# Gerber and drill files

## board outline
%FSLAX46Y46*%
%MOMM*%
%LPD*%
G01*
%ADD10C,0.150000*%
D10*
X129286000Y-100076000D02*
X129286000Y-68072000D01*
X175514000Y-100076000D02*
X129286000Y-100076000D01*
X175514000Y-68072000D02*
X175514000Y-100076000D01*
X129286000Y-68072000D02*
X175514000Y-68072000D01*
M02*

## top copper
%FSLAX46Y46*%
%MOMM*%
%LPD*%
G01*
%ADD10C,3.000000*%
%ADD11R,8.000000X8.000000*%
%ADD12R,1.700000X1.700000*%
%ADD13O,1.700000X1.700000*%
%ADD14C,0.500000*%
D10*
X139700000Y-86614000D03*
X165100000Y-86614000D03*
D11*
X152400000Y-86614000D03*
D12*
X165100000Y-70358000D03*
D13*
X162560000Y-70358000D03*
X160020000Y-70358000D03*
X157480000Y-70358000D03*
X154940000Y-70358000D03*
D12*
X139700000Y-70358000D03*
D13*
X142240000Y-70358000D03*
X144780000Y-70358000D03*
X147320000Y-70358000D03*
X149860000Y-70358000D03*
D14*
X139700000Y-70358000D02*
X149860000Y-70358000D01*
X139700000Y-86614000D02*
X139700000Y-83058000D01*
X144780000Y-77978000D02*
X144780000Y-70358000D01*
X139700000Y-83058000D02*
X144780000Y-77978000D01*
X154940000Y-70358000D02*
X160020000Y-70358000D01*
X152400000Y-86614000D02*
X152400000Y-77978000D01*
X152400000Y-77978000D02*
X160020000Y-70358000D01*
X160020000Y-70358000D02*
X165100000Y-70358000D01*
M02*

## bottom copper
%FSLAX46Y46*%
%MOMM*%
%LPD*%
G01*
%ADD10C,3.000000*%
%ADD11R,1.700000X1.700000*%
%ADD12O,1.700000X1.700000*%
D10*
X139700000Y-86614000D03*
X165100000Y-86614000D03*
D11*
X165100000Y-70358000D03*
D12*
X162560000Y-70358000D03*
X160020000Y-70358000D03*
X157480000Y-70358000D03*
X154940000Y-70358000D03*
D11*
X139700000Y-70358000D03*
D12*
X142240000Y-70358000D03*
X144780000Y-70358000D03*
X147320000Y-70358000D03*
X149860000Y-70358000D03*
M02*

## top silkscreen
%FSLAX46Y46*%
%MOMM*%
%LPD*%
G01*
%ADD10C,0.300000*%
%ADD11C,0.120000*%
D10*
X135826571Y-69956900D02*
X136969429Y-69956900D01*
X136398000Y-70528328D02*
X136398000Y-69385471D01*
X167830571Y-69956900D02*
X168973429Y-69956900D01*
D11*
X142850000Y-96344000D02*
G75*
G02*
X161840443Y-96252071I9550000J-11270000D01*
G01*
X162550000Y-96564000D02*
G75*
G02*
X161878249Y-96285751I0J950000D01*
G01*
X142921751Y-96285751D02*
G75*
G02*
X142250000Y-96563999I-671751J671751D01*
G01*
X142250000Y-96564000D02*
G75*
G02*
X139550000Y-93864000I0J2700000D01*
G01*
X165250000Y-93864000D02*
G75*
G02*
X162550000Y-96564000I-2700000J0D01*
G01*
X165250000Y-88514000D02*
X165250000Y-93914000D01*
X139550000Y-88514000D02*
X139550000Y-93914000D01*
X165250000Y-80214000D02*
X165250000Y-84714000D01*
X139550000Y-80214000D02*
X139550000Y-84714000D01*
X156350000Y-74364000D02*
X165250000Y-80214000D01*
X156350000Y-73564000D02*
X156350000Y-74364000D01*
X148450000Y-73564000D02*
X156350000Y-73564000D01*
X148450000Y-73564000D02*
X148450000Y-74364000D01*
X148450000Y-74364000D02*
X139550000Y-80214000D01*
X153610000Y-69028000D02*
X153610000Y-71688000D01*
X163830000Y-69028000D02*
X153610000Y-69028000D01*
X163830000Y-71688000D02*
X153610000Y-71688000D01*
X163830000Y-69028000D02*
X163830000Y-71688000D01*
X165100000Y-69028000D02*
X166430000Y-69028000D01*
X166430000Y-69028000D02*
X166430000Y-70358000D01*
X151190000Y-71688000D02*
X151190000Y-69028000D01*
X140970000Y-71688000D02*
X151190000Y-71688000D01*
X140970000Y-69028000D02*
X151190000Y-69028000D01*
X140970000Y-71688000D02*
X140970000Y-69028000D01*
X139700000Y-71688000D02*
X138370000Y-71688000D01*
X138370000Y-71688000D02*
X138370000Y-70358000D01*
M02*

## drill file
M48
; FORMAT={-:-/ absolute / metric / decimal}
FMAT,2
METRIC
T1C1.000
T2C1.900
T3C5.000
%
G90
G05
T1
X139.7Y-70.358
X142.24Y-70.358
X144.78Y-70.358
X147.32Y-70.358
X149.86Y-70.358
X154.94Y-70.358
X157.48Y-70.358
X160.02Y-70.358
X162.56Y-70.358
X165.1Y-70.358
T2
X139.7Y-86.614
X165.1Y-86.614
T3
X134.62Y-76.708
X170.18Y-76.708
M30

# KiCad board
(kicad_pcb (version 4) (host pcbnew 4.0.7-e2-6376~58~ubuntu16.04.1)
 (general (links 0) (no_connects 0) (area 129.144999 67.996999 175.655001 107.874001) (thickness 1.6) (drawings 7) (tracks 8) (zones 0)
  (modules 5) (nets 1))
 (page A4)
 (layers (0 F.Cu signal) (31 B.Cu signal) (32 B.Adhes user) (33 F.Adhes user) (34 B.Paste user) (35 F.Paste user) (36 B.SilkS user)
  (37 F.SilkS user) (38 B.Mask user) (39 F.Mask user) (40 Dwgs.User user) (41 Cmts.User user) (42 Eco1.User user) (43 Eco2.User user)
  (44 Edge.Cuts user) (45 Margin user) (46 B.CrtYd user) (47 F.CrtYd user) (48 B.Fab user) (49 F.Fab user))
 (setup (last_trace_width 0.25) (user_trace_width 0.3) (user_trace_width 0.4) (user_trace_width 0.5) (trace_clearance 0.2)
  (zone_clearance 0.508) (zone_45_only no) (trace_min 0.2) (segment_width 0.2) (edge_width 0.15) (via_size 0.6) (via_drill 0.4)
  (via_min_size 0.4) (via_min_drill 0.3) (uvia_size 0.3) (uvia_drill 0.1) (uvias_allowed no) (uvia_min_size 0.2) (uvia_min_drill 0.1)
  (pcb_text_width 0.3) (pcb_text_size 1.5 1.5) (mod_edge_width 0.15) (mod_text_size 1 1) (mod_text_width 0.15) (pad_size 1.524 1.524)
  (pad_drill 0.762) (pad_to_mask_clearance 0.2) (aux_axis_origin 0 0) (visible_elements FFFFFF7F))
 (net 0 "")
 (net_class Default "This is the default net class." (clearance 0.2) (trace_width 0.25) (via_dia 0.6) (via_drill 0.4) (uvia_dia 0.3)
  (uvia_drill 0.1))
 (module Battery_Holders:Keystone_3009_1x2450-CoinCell (layer F.Cu) (at 152.4 86.614)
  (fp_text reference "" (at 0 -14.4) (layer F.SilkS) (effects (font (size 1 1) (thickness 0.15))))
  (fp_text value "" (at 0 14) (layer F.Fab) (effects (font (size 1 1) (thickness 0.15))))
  (fp_arc (start 0 21) (end -9.55 9.73) (angle 80) (layer F.SilkS) (width 0.12))
  (fp_arc (start 10.15 9) (end 10.15 9.95) (angle 45) (layer F.SilkS) (width 0.12))
  (fp_arc (start -10.15 9) (end -10.15 9.95) (angle -45) (layer F.SilkS) (width 0.12))
  (fp_arc (start -10.15 7.25) (end -10.15 9.95) (angle 90) (layer F.SilkS) (width 0.12))
  (fp_arc (start 10.15 7.25) (end 10.15 9.95) (angle -90) (layer F.SilkS) (width 0.12))
  (fp_line (start 12.85 1.9) (end 12.85 7.3) (layer F.SilkS) (width 0.12))
  (fp_line (start -12.85 1.9) (end -12.85 7.3) (layer F.SilkS) (width 0.12))
  (fp_line (start 12.85 -6.4) (end 12.85 -1.9) (layer F.SilkS) (width 0.12))
  (fp_line (start -12.85 -6.4) (end -12.85 -1.9) (layer F.SilkS) (width 0.12))
  (fp_line (start 3.95 -12.25) (end 12.85 -6.4) (layer F.SilkS) (width 0.12))
  (fp_line (start 3.95 -13.05) (end 3.95 -12.25) (layer F.SilkS) (width 0.12))
  (fp_line (start -3.95 -13.05) (end 3.95 -13.05) (layer F.SilkS) (width 0.12))
  (fp_line (start -3.95 -13.05) (end -3.95 -12.25) (layer F.SilkS) (width 0.12))
  (fp_line (start -3.95 -12.25) (end -12.85 -6.4) (layer F.SilkS) (width 0.12))
  (pad 1 thru_hole circle (at -12.7 0) (size 3 3) (drill 1.9) (layers *.Cu *.Mask))
  (pad 1 thru_hole circle (at 12.7 0) (size 3 3) (drill 1.9) (layers *.Cu *.Mask)) (pad 2 smd rect (at 0 0) (size 8 8) (layers F.Cu F.Mask)))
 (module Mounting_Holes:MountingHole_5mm (layer F.Cu) (at 170.18 76.708)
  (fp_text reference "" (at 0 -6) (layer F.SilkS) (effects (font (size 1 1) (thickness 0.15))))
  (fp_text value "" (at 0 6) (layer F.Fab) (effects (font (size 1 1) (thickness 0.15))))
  (pad 1 np_thru_hole circle (at 0 0) (size 5 5) (drill 5) (layers *.Cu *.Mask)))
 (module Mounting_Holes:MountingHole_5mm (layer F.Cu) (at 134.62 76.708)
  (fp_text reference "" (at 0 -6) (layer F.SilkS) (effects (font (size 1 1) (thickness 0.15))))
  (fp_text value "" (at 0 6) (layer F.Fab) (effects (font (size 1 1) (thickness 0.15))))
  (pad 1 np_thru_hole circle (at 0 0) (size 5 5) (drill 5) (layers *.Cu *.Mask)))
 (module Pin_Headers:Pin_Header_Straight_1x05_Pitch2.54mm (layer F.Cu) (at 165.1 70.358 270)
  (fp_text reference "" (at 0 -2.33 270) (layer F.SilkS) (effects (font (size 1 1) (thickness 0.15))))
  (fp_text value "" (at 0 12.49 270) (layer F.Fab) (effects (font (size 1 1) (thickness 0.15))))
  (fp_line (start -1.33 11.49) (end 1.33 11.49) (layer F.SilkS) (width 0.12))
  (fp_line (start -1.33 1.27) (end -1.33 11.49) (layer F.SilkS) (width 0.12))
  (fp_line (start 1.33 1.27) (end 1.33 11.49) (layer F.SilkS) (width 0.12))
  (fp_line (start -1.33 1.27) (end 1.33 1.27) (layer F.SilkS) (width 0.12))
  (fp_line (start -1.33 0) (end -1.33 -1.33) (layer F.SilkS) (width 0.12))
  (fp_line (start -1.33 -1.33) (end 0 -1.33) (layer F.SilkS) (width 0.12))
  (pad 1 thru_hole rect (at 0 0 270) (size 1.7 1.7) (drill 1) (layers *.Cu *.Mask))
  (pad 2 thru_hole oval (at 0 2.54 270) (size 1.7 1.7) (drill 1) (layers *.Cu *.Mask))
  (pad 3 thru_hole oval (at 0 5.08 270) (size 1.7 1.7) (drill 1) (layers *.Cu *.Mask))
  (pad 4 thru_hole oval (at 0 7.62 270) (size 1.7 1.7) (drill 1) (layers *.Cu *.Mask))
  (pad 5 thru_hole oval (at 0 10.16 270) (size 1.7 1.7) (drill 1) (layers *.Cu *.Mask)))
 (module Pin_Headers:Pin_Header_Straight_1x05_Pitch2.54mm (layer F.Cu) (at 139.7 70.358 90)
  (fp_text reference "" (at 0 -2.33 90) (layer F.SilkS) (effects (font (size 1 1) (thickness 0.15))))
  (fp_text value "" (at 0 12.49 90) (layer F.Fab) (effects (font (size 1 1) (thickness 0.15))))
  (fp_line (start -1.33 11.49) (end 1.33 11.49) (layer F.SilkS) (width 0.12))
  (fp_line (start -1.33 1.27) (end -1.33 11.49) (layer F.SilkS) (width 0.12))
  (fp_line (start 1.33 1.27) (end 1.33 11.49) (layer F.SilkS) (width 0.12))
  (fp_line (start -1.33 1.27) (end 1.33 1.27) (layer F.SilkS) (width 0.12))
  (fp_line (start -1.33 0) (end -1.33 -1.33) (layer F.SilkS) (width 0.12))
  (fp_line (start -1.33 -1.33) (end 0 -1.33) (layer F.SilkS) (width 0.12))
  (pad 1 thru_hole rect (at 0 0 90) (size 1.7 1.7) (drill 1) (layers *.Cu *.Mask))
  (pad 2 thru_hole oval (at 0 2.54 90) (size 1.7 1.7) (drill 1) (layers *.Cu *.Mask))
  (pad 3 thru_hole oval (at 0 5.08 90) (size 1.7 1.7) (drill 1) (layers *.Cu *.Mask))
  (pad 4 thru_hole oval (at 0 7.62 90) (size 1.7 1.7) (drill 1) (layers *.Cu *.Mask))
  (pad 5 thru_hole oval (at 0 10.16 90) (size 1.7 1.7) (drill 1) (layers *.Cu *.Mask)))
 (gr_line (start 129.286 100.076) (end 129.286 68.072) (angle 90) (layer Edge.Cuts) (width 0.15))
 (gr_line (start 175.514 100.076) (end 129.286 100.076) (angle 90) (layer Edge.Cuts) (width 0.15))
 (gr_line (start 175.514 68.072) (end 175.514 100.076) (angle 90) (layer Edge.Cuts) (width 0.15))
 (gr_line (start 129.286 68.072) (end 175.514 68.072) (angle 90) (layer Edge.Cuts) (width 0.15))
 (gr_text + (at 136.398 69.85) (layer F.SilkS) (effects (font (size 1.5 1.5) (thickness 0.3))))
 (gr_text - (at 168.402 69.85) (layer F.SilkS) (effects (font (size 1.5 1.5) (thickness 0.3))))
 (segment (start 139.7 70.358) (end 149.86 70.358) (width 0.5) (layer F.Cu) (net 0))
 (segment (start 139.7 86.614) (end 139.7 83.058) (width 0.5) (layer F.Cu) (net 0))
 (segment (start 144.78 77.978) (end 144.78 70.358) (width 0.5) (layer F.Cu) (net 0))
 (segment (start 139.7 83.058) (end 144.78 77.978) (width 0.5) (layer F.Cu) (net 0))
 (segment (start 154.94 70.358) (end 160.02 70.358) (width 0.5) (layer F.Cu) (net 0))
 (segment (start 152.4 86.614) (end 152.4 77.978) (width 0.5) (layer F.Cu) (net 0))
 (segment (start 152.4 77.978) (end 160.02 70.358) (width 0.5) (layer F.Cu) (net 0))
 (segment (start 160.02 70.358) (end 165.1 70.358) (width 0.5) (layer F.Cu) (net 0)))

